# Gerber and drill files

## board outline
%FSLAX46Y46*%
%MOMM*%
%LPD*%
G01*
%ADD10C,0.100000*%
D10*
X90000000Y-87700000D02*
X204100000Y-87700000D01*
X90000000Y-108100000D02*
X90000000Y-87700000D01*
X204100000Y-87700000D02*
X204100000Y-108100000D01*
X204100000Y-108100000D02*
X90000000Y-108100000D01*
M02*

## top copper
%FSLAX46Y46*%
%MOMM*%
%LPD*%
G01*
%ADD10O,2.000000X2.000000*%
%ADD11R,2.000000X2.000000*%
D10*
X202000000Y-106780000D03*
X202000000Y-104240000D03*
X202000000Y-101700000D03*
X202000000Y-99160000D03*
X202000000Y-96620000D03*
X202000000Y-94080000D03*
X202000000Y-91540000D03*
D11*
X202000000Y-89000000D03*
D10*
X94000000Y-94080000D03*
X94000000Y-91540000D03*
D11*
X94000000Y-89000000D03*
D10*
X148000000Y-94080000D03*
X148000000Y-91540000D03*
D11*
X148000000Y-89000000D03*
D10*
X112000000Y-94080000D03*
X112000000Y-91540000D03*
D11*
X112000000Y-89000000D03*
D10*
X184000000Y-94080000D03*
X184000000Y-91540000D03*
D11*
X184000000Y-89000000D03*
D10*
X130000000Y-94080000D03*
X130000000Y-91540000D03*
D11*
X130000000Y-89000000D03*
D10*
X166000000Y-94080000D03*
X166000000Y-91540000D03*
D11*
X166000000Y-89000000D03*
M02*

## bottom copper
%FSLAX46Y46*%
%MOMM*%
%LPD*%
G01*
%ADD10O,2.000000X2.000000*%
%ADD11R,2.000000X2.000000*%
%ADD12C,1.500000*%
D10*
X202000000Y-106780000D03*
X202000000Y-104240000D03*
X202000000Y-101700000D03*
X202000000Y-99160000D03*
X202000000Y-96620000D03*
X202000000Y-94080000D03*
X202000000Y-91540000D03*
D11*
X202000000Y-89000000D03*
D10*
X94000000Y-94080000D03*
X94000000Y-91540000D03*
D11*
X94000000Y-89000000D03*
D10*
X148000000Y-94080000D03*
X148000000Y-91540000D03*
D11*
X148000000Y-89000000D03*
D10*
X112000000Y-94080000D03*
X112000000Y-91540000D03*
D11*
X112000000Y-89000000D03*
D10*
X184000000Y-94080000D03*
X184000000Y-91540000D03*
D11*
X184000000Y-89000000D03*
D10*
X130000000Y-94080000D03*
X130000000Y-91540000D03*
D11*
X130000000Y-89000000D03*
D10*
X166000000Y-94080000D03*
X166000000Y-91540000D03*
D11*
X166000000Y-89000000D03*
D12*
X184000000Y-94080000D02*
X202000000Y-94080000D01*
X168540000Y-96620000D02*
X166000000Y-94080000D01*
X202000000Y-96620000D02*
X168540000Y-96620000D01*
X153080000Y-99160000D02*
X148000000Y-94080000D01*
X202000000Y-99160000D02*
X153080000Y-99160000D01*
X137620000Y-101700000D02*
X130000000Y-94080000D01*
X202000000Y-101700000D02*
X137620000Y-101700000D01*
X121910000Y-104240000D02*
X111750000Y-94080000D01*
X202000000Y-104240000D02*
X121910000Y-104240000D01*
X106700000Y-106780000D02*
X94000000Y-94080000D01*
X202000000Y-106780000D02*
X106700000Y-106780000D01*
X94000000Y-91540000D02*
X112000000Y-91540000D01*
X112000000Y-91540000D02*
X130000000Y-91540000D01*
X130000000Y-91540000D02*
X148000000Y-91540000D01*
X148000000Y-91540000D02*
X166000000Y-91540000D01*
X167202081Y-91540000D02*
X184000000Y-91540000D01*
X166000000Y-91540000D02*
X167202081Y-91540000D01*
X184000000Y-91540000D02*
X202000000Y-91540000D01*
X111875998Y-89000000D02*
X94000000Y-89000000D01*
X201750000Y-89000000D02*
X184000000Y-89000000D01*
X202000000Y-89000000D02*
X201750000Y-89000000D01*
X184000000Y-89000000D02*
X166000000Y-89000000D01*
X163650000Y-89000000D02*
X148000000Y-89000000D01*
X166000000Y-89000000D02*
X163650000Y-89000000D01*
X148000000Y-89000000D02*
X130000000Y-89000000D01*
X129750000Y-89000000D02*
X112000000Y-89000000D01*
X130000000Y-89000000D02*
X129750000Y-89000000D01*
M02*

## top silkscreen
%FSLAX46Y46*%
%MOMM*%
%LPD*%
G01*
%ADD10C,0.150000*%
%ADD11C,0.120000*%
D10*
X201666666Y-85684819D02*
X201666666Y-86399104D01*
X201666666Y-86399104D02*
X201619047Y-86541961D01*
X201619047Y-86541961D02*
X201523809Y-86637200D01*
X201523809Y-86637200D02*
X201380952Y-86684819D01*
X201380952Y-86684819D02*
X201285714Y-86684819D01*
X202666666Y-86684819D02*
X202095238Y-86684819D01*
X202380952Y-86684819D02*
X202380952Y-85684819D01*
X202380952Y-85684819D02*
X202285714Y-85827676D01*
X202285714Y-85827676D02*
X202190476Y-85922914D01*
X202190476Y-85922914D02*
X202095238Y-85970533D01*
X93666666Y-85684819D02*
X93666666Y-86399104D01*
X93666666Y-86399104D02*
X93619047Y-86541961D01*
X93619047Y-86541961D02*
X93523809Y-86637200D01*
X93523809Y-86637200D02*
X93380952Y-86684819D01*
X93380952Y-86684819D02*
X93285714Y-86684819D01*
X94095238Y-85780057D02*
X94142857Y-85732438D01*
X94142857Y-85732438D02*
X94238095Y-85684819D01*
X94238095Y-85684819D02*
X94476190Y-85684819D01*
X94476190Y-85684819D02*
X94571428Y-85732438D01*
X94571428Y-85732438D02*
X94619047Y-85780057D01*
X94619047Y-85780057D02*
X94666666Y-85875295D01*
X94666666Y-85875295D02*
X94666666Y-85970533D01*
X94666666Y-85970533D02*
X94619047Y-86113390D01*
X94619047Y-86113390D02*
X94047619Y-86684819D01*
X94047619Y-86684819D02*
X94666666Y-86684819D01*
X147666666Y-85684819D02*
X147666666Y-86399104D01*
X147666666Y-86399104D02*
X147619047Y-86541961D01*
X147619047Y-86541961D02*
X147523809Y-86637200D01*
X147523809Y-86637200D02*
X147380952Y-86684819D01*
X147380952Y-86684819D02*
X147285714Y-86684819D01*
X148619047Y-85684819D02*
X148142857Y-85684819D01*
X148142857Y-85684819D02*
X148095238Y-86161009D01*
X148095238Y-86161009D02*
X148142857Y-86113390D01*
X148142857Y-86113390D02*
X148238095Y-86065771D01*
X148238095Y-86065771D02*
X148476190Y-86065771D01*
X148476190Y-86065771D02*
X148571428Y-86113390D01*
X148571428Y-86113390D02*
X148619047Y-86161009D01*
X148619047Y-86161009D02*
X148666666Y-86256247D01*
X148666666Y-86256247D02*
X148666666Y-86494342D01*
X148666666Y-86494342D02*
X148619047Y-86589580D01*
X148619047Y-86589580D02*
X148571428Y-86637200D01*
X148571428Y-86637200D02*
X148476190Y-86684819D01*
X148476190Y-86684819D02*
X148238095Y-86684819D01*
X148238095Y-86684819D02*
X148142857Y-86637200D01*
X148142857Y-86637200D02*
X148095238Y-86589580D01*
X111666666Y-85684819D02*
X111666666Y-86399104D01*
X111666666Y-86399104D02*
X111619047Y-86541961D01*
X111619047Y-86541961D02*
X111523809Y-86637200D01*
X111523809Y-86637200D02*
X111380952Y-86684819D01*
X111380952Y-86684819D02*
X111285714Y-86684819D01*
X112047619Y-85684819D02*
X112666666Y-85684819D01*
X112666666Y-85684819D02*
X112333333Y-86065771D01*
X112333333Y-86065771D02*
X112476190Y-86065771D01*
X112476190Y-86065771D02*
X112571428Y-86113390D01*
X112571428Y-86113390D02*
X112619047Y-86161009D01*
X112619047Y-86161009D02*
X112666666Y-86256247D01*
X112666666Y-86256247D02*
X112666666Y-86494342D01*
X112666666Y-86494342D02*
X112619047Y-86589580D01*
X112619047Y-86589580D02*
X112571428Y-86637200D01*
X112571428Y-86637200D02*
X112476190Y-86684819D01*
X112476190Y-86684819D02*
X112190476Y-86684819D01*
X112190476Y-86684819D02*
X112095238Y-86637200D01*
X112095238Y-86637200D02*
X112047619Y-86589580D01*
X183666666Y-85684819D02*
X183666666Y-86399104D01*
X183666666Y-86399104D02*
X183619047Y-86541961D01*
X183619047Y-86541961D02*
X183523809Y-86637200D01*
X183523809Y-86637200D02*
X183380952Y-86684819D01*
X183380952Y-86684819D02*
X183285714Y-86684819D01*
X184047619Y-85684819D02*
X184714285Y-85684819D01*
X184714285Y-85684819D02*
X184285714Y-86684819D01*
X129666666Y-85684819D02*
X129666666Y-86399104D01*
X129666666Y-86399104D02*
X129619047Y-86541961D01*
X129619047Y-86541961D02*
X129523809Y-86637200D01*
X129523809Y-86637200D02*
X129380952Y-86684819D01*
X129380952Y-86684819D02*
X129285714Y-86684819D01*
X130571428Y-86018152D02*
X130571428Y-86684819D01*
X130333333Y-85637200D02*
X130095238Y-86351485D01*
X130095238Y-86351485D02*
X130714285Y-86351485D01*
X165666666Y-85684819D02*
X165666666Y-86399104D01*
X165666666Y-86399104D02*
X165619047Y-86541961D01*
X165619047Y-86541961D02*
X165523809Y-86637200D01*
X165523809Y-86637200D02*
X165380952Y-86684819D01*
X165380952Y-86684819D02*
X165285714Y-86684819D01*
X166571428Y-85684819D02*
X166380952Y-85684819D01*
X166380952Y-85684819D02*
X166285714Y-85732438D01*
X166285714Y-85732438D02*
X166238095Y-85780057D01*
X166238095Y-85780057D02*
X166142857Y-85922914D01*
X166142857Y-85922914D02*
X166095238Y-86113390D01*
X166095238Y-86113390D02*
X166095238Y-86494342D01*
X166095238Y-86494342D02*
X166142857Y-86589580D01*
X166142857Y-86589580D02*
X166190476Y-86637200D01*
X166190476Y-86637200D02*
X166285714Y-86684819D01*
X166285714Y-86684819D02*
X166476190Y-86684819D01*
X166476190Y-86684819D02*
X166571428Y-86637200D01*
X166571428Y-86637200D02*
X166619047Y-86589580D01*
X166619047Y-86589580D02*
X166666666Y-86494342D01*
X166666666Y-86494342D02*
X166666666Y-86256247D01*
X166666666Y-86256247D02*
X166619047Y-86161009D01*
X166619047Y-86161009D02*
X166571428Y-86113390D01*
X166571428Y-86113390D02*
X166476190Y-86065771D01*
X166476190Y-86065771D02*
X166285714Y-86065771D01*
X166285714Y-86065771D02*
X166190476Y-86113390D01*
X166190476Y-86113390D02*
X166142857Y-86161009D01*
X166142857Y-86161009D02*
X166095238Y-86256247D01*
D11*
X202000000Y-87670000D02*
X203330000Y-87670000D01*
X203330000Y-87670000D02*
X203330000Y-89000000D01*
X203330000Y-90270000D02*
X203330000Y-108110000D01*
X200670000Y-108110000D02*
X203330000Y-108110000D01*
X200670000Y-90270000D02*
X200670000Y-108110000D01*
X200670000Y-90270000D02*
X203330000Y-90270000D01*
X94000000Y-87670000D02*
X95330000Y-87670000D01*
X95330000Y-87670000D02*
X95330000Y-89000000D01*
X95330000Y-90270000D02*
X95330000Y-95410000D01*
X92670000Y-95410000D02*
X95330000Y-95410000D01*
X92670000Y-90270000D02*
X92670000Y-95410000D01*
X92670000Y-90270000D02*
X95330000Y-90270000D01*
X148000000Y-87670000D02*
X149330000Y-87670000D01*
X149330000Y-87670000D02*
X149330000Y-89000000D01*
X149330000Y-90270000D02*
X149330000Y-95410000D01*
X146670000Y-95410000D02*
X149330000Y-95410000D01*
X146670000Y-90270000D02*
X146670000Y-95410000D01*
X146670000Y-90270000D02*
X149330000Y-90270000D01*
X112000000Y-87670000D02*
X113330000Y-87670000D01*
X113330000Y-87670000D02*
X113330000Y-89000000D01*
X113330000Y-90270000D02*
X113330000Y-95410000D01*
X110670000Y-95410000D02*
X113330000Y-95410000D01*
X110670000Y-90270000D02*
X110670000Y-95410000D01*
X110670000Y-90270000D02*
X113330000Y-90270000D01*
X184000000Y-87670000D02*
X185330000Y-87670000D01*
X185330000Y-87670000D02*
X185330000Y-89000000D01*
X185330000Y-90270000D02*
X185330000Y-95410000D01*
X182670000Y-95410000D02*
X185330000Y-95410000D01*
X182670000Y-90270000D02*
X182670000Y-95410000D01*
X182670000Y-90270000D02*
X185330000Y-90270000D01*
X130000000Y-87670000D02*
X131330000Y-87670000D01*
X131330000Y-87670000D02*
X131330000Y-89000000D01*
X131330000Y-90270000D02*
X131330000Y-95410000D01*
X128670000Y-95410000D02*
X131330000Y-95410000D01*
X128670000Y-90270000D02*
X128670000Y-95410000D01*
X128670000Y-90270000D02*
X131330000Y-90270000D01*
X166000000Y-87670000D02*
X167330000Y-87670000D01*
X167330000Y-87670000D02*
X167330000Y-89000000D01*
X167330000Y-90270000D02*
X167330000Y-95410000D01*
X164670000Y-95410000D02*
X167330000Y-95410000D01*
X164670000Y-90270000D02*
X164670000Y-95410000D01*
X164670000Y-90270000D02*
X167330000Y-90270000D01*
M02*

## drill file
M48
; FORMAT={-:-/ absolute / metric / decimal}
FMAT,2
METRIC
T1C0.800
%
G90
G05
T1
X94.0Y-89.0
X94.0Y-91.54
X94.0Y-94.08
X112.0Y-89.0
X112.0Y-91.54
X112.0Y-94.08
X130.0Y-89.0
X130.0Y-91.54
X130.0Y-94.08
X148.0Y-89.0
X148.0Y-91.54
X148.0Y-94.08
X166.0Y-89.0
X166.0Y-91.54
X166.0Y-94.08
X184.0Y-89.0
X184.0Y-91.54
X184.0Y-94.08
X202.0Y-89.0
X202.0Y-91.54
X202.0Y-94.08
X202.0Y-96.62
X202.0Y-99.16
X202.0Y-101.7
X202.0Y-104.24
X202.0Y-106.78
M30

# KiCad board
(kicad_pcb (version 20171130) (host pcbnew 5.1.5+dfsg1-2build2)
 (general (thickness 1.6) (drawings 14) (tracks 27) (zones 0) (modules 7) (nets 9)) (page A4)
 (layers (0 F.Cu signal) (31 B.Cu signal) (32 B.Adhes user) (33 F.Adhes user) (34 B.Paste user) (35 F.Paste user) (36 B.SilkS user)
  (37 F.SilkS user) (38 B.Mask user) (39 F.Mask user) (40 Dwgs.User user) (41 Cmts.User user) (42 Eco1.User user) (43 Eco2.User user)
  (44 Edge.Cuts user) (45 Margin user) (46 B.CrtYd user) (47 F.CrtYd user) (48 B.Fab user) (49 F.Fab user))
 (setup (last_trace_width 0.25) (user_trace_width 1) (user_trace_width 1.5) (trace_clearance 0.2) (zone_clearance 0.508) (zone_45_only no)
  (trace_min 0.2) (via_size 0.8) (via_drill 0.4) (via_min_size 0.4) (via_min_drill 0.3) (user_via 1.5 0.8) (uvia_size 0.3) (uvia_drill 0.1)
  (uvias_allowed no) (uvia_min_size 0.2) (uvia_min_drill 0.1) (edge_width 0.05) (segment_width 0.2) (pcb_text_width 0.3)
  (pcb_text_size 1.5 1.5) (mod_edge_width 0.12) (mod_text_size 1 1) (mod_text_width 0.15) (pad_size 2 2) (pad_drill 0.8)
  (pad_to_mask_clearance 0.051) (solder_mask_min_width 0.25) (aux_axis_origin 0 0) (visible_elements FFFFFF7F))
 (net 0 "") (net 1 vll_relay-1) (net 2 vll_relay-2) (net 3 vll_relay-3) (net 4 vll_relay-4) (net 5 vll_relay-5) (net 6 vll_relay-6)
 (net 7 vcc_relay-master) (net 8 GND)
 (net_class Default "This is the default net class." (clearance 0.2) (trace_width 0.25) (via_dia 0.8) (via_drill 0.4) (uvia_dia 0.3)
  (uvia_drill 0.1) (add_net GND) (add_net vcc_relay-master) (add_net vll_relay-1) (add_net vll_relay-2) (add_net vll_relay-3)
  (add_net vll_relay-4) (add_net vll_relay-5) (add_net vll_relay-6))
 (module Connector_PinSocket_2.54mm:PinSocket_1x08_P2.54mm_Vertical (layer F.Cu) (at 202 89)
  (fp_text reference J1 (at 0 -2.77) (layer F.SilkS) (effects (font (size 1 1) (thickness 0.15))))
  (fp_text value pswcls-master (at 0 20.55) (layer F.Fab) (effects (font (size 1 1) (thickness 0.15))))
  (fp_line (start 0 -1.33) (end 1.33 -1.33) (layer F.SilkS) (width 0.12))
  (fp_line (start 1.33 -1.33) (end 1.33 0) (layer F.SilkS) (width 0.12))
  (fp_line (start 1.33 1.27) (end 1.33 19.11) (layer F.SilkS) (width 0.12))
  (fp_line (start -1.33 19.11) (end 1.33 19.11) (layer F.SilkS) (width 0.12))
  (fp_line (start -1.33 1.27) (end -1.33 19.11) (layer F.SilkS) (width 0.12))
  (fp_line (start -1.33 1.27) (end 1.33 1.27) (layer F.SilkS) (width 0.12))
  (pad 8 thru_hole oval (at 0 17.78) (size 2 2) (drill 0.8) (layers *.Cu *.Mask) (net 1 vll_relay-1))
  (pad 7 thru_hole oval (at 0 15.24) (size 2 2) (drill 0.8) (layers *.Cu *.Mask) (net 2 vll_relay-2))
  (pad 6 thru_hole oval (at 0 12.7) (size 2 2) (drill 0.8) (layers *.Cu *.Mask) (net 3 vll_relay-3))
  (pad 5 thru_hole oval (at 0 10.16) (size 2 2) (drill 0.8) (layers *.Cu *.Mask) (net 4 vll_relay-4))
  (pad 4 thru_hole oval (at 0 7.62) (size 2 2) (drill 0.8) (layers *.Cu *.Mask) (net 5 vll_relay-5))
  (pad 3 thru_hole oval (at 0 5.08) (size 2 2) (drill 0.8) (layers *.Cu *.Mask) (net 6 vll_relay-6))
  (pad 2 thru_hole oval (at 0 2.54) (size 2 2) (drill 0.8) (layers *.Cu *.Mask) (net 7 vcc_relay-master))
  (pad 1 thru_hole rect (at 0 0) (size 2 2) (drill 0.8) (layers *.Cu *.Mask) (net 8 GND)))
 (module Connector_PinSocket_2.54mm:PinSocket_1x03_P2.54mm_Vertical (layer F.Cu) (at 94 89)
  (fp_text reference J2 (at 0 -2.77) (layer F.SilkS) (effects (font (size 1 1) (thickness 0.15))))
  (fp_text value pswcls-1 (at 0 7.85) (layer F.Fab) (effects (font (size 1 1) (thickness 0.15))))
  (fp_line (start 0 -1.33) (end 1.33 -1.33) (layer F.SilkS) (width 0.12))
  (fp_line (start 1.33 -1.33) (end 1.33 0) (layer F.SilkS) (width 0.12))
  (fp_line (start 1.33 1.27) (end 1.33 6.41) (layer F.SilkS) (width 0.12))
  (fp_line (start -1.33 6.41) (end 1.33 6.41) (layer F.SilkS) (width 0.12))
  (fp_line (start -1.33 1.27) (end -1.33 6.41) (layer F.SilkS) (width 0.12))
  (fp_line (start -1.33 1.27) (end 1.33 1.27) (layer F.SilkS) (width 0.12))
  (pad 3 thru_hole oval (at 0 5.08) (size 2 2) (drill 0.8) (layers *.Cu *.Mask) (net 1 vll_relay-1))
  (pad 2 thru_hole oval (at 0 2.54) (size 2 2) (drill 0.8) (layers *.Cu *.Mask) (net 7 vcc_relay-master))
  (pad 1 thru_hole rect (at 0 0) (size 2 2) (drill 0.8) (layers *.Cu *.Mask) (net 8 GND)))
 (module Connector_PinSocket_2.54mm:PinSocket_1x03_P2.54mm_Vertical (layer F.Cu) (at 148 89)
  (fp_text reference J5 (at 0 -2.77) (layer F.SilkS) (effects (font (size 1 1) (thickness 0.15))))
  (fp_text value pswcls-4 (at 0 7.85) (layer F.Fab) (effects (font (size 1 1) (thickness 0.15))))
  (fp_line (start 0 -1.33) (end 1.33 -1.33) (layer F.SilkS) (width 0.12))
  (fp_line (start 1.33 -1.33) (end 1.33 0) (layer F.SilkS) (width 0.12))
  (fp_line (start 1.33 1.27) (end 1.33 6.41) (layer F.SilkS) (width 0.12))
  (fp_line (start -1.33 6.41) (end 1.33 6.41) (layer F.SilkS) (width 0.12))
  (fp_line (start -1.33 1.27) (end -1.33 6.41) (layer F.SilkS) (width 0.12))
  (fp_line (start -1.33 1.27) (end 1.33 1.27) (layer F.SilkS) (width 0.12))
  (pad 3 thru_hole oval (at 0 5.08) (size 2 2) (drill 0.8) (layers *.Cu *.Mask) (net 4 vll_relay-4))
  (pad 2 thru_hole oval (at 0 2.54) (size 2 2) (drill 0.8) (layers *.Cu *.Mask) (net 7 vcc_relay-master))
  (pad 1 thru_hole rect (at 0 0) (size 2 2) (drill 0.8) (layers *.Cu *.Mask) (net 8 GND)))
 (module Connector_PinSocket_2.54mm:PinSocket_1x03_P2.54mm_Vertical (layer F.Cu) (at 112 89)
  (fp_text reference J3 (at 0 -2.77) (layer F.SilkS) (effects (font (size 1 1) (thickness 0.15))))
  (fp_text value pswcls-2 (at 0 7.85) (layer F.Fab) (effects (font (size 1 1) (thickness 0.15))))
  (fp_line (start 0 -1.33) (end 1.33 -1.33) (layer F.SilkS) (width 0.12))
  (fp_line (start 1.33 -1.33) (end 1.33 0) (layer F.SilkS) (width 0.12))
  (fp_line (start 1.33 1.27) (end 1.33 6.41) (layer F.SilkS) (width 0.12))
  (fp_line (start -1.33 6.41) (end 1.33 6.41) (layer F.SilkS) (width 0.12))
  (fp_line (start -1.33 1.27) (end -1.33 6.41) (layer F.SilkS) (width 0.12))
  (fp_line (start -1.33 1.27) (end 1.33 1.27) (layer F.SilkS) (width 0.12))
  (pad 3 thru_hole oval (at 0 5.08) (size 2 2) (drill 0.8) (layers *.Cu *.Mask) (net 2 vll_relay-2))
  (pad 2 thru_hole oval (at 0 2.54) (size 2 2) (drill 0.8) (layers *.Cu *.Mask) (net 7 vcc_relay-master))
  (pad 1 thru_hole rect (at 0 0) (size 2 2) (drill 0.8) (layers *.Cu *.Mask) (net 8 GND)))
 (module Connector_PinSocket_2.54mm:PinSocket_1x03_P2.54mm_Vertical (layer F.Cu) (at 184 89)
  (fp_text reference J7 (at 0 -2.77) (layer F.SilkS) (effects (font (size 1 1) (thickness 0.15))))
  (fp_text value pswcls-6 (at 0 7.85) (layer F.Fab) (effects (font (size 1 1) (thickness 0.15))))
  (fp_line (start 0 -1.33) (end 1.33 -1.33) (layer F.SilkS) (width 0.12))
  (fp_line (start 1.33 -1.33) (end 1.33 0) (layer F.SilkS) (width 0.12))
  (fp_line (start 1.33 1.27) (end 1.33 6.41) (layer F.SilkS) (width 0.12))
  (fp_line (start -1.33 6.41) (end 1.33 6.41) (layer F.SilkS) (width 0.12))
  (fp_line (start -1.33 1.27) (end -1.33 6.41) (layer F.SilkS) (width 0.12))
  (fp_line (start -1.33 1.27) (end 1.33 1.27) (layer F.SilkS) (width 0.12))
  (pad 3 thru_hole oval (at 0 5.08) (size 2 2) (drill 0.8) (layers *.Cu *.Mask) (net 6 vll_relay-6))
  (pad 2 thru_hole oval (at 0 2.54) (size 2 2) (drill 0.8) (layers *.Cu *.Mask) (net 7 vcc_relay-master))
  (pad 1 thru_hole rect (at 0 0) (size 2 2) (drill 0.8) (layers *.Cu *.Mask) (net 8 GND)))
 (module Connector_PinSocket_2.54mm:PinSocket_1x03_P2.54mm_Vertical (layer F.Cu) (at 130 89)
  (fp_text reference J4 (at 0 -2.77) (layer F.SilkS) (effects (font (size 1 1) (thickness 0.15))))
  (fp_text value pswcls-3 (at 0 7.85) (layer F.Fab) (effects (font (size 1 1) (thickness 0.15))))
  (fp_line (start 0 -1.33) (end 1.33 -1.33) (layer F.SilkS) (width 0.12))
  (fp_line (start 1.33 -1.33) (end 1.33 0) (layer F.SilkS) (width 0.12))
  (fp_line (start 1.33 1.27) (end 1.33 6.41) (layer F.SilkS) (width 0.12))
  (fp_line (start -1.33 6.41) (end 1.33 6.41) (layer F.SilkS) (width 0.12))
  (fp_line (start -1.33 1.27) (end -1.33 6.41) (layer F.SilkS) (width 0.12))
  (fp_line (start -1.33 1.27) (end 1.33 1.27) (layer F.SilkS) (width 0.12))
  (pad 3 thru_hole oval (at 0 5.08) (size 2 2) (drill 0.8) (layers *.Cu *.Mask) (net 3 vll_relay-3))
  (pad 2 thru_hole oval (at 0 2.54) (size 2 2) (drill 0.8) (layers *.Cu *.Mask) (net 7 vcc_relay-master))
  (pad 1 thru_hole rect (at 0 0) (size 2 2) (drill 0.8) (layers *.Cu *.Mask) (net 8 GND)))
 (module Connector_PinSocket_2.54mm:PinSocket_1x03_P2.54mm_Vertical (layer F.Cu) (at 166 89)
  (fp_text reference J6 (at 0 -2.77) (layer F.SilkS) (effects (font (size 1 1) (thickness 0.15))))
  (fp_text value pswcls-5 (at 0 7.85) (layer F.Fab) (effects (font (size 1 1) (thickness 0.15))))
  (fp_line (start 0 -1.33) (end 1.33 -1.33) (layer F.SilkS) (width 0.12))
  (fp_line (start 1.33 -1.33) (end 1.33 0) (layer F.SilkS) (width 0.12))
  (fp_line (start 1.33 1.27) (end 1.33 6.41) (layer F.SilkS) (width 0.12))
  (fp_line (start -1.33 6.41) (end 1.33 6.41) (layer F.SilkS) (width 0.12))
  (fp_line (start -1.33 1.27) (end -1.33 6.41) (layer F.SilkS) (width 0.12))
  (fp_line (start -1.33 1.27) (end 1.33 1.27) (layer F.SilkS) (width 0.12))
  (pad 3 thru_hole oval (at 0 5.08) (size 2 2) (drill 0.8) (layers *.Cu *.Mask) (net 5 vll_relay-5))
  (pad 2 thru_hole oval (at 0 2.54) (size 2 2) (drill 0.8) (layers *.Cu *.Mask) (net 7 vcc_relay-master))
  (pad 1 thru_hole rect (at 0 0) (size 2 2) (drill 0.8) (layers *.Cu *.Mask) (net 8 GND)))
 (gr_line (start 90 87.7) (end 204.1 87.7) (layer Edge.Cuts) (width 0.1))
 (gr_line (start 90 108.1) (end 90 87.7) (layer Edge.Cuts) (width 0.1))
 (gr_line (start 204.1 87.7) (end 204.1 108.1) (layer Edge.Cuts) (width 0.1))
 (gr_line (start 204.1 108.1) (end 90 108.1) (layer Edge.Cuts) (width 0.1))
 (segment (start 184 94.08) (end 202 94.08) (width 1.5) (layer B.Cu) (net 6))
 (segment (start 168.54 96.62) (end 166 94.08) (width 1.5) (layer B.Cu) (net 5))
 (segment (start 202 96.62) (end 168.54 96.62) (width 1.5) (layer B.Cu) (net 5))
 (segment (start 153.08 99.16) (end 148 94.08) (width 1.5) (layer B.Cu) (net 4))
 (segment (start 202 99.16) (end 153.08 99.16) (width 1.5) (layer B.Cu) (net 4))
 (segment (start 137.62 101.7) (end 130 94.08) (width 1.5) (layer B.Cu) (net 3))
 (segment (start 202 101.7) (end 137.62 101.7) (width 1.5) (layer B.Cu) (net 3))
 (segment (start 121.91 104.24) (end 111.75 94.08) (width 1.5) (layer B.Cu) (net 2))
 (segment (start 202 104.24) (end 121.91 104.24) (width 1.5) (layer B.Cu) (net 2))
 (segment (start 106.7 106.78) (end 94 94.08) (width 1.5) (layer B.Cu) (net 1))
 (segment (start 202 106.78) (end 106.7 106.78) (width 1.5) (layer B.Cu) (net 1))
 (segment (start 94 91.54) (end 112 91.54) (width 1.5) (layer B.Cu) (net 7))
 (segment (start 112 91.54) (end 130 91.54) (width 1.5) (layer B.Cu) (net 7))
 (segment (start 130 91.54) (end 148 91.54) (width 1.5) (layer B.Cu) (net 7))
 (segment (start 148 91.54) (end 166 91.54) (width 1.5) (layer B.Cu) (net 7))
 (segment (start 167.202081 91.54) (end 184 91.54) (width 1.5) (layer B.Cu) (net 7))
 (segment (start 166 91.54) (end 167.202081 91.54) (width 1.5) (layer B.Cu) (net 7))
 (segment (start 184 91.54) (end 202 91.54) (width 1.5) (layer B.Cu) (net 7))
 (segment (start 111.875998 89) (end 94 89) (width 1.5) (layer B.Cu) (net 8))
 (segment (start 201.75 89) (end 184 89) (width 1.5) (layer B.Cu) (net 8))
 (segment (start 202 89) (end 201.75 89) (width 1.5) (layer B.Cu) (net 8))
 (segment (start 184 89) (end 166 89) (width 1.5) (layer B.Cu) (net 8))
 (segment (start 163.65 89) (end 148 89) (width 1.5) (layer B.Cu) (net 8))
 (segment (start 166 89) (end 163.65 89) (width 1.5) (layer B.Cu) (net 8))
 (segment (start 148 89) (end 130 89) (width 1.5) (layer B.Cu) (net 8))
 (segment (start 129.75 89) (end 112 89) (width 1.5) (layer B.Cu) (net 8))
 (segment (start 130 89) (end 129.75 89) (width 1.5) (layer B.Cu) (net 8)))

